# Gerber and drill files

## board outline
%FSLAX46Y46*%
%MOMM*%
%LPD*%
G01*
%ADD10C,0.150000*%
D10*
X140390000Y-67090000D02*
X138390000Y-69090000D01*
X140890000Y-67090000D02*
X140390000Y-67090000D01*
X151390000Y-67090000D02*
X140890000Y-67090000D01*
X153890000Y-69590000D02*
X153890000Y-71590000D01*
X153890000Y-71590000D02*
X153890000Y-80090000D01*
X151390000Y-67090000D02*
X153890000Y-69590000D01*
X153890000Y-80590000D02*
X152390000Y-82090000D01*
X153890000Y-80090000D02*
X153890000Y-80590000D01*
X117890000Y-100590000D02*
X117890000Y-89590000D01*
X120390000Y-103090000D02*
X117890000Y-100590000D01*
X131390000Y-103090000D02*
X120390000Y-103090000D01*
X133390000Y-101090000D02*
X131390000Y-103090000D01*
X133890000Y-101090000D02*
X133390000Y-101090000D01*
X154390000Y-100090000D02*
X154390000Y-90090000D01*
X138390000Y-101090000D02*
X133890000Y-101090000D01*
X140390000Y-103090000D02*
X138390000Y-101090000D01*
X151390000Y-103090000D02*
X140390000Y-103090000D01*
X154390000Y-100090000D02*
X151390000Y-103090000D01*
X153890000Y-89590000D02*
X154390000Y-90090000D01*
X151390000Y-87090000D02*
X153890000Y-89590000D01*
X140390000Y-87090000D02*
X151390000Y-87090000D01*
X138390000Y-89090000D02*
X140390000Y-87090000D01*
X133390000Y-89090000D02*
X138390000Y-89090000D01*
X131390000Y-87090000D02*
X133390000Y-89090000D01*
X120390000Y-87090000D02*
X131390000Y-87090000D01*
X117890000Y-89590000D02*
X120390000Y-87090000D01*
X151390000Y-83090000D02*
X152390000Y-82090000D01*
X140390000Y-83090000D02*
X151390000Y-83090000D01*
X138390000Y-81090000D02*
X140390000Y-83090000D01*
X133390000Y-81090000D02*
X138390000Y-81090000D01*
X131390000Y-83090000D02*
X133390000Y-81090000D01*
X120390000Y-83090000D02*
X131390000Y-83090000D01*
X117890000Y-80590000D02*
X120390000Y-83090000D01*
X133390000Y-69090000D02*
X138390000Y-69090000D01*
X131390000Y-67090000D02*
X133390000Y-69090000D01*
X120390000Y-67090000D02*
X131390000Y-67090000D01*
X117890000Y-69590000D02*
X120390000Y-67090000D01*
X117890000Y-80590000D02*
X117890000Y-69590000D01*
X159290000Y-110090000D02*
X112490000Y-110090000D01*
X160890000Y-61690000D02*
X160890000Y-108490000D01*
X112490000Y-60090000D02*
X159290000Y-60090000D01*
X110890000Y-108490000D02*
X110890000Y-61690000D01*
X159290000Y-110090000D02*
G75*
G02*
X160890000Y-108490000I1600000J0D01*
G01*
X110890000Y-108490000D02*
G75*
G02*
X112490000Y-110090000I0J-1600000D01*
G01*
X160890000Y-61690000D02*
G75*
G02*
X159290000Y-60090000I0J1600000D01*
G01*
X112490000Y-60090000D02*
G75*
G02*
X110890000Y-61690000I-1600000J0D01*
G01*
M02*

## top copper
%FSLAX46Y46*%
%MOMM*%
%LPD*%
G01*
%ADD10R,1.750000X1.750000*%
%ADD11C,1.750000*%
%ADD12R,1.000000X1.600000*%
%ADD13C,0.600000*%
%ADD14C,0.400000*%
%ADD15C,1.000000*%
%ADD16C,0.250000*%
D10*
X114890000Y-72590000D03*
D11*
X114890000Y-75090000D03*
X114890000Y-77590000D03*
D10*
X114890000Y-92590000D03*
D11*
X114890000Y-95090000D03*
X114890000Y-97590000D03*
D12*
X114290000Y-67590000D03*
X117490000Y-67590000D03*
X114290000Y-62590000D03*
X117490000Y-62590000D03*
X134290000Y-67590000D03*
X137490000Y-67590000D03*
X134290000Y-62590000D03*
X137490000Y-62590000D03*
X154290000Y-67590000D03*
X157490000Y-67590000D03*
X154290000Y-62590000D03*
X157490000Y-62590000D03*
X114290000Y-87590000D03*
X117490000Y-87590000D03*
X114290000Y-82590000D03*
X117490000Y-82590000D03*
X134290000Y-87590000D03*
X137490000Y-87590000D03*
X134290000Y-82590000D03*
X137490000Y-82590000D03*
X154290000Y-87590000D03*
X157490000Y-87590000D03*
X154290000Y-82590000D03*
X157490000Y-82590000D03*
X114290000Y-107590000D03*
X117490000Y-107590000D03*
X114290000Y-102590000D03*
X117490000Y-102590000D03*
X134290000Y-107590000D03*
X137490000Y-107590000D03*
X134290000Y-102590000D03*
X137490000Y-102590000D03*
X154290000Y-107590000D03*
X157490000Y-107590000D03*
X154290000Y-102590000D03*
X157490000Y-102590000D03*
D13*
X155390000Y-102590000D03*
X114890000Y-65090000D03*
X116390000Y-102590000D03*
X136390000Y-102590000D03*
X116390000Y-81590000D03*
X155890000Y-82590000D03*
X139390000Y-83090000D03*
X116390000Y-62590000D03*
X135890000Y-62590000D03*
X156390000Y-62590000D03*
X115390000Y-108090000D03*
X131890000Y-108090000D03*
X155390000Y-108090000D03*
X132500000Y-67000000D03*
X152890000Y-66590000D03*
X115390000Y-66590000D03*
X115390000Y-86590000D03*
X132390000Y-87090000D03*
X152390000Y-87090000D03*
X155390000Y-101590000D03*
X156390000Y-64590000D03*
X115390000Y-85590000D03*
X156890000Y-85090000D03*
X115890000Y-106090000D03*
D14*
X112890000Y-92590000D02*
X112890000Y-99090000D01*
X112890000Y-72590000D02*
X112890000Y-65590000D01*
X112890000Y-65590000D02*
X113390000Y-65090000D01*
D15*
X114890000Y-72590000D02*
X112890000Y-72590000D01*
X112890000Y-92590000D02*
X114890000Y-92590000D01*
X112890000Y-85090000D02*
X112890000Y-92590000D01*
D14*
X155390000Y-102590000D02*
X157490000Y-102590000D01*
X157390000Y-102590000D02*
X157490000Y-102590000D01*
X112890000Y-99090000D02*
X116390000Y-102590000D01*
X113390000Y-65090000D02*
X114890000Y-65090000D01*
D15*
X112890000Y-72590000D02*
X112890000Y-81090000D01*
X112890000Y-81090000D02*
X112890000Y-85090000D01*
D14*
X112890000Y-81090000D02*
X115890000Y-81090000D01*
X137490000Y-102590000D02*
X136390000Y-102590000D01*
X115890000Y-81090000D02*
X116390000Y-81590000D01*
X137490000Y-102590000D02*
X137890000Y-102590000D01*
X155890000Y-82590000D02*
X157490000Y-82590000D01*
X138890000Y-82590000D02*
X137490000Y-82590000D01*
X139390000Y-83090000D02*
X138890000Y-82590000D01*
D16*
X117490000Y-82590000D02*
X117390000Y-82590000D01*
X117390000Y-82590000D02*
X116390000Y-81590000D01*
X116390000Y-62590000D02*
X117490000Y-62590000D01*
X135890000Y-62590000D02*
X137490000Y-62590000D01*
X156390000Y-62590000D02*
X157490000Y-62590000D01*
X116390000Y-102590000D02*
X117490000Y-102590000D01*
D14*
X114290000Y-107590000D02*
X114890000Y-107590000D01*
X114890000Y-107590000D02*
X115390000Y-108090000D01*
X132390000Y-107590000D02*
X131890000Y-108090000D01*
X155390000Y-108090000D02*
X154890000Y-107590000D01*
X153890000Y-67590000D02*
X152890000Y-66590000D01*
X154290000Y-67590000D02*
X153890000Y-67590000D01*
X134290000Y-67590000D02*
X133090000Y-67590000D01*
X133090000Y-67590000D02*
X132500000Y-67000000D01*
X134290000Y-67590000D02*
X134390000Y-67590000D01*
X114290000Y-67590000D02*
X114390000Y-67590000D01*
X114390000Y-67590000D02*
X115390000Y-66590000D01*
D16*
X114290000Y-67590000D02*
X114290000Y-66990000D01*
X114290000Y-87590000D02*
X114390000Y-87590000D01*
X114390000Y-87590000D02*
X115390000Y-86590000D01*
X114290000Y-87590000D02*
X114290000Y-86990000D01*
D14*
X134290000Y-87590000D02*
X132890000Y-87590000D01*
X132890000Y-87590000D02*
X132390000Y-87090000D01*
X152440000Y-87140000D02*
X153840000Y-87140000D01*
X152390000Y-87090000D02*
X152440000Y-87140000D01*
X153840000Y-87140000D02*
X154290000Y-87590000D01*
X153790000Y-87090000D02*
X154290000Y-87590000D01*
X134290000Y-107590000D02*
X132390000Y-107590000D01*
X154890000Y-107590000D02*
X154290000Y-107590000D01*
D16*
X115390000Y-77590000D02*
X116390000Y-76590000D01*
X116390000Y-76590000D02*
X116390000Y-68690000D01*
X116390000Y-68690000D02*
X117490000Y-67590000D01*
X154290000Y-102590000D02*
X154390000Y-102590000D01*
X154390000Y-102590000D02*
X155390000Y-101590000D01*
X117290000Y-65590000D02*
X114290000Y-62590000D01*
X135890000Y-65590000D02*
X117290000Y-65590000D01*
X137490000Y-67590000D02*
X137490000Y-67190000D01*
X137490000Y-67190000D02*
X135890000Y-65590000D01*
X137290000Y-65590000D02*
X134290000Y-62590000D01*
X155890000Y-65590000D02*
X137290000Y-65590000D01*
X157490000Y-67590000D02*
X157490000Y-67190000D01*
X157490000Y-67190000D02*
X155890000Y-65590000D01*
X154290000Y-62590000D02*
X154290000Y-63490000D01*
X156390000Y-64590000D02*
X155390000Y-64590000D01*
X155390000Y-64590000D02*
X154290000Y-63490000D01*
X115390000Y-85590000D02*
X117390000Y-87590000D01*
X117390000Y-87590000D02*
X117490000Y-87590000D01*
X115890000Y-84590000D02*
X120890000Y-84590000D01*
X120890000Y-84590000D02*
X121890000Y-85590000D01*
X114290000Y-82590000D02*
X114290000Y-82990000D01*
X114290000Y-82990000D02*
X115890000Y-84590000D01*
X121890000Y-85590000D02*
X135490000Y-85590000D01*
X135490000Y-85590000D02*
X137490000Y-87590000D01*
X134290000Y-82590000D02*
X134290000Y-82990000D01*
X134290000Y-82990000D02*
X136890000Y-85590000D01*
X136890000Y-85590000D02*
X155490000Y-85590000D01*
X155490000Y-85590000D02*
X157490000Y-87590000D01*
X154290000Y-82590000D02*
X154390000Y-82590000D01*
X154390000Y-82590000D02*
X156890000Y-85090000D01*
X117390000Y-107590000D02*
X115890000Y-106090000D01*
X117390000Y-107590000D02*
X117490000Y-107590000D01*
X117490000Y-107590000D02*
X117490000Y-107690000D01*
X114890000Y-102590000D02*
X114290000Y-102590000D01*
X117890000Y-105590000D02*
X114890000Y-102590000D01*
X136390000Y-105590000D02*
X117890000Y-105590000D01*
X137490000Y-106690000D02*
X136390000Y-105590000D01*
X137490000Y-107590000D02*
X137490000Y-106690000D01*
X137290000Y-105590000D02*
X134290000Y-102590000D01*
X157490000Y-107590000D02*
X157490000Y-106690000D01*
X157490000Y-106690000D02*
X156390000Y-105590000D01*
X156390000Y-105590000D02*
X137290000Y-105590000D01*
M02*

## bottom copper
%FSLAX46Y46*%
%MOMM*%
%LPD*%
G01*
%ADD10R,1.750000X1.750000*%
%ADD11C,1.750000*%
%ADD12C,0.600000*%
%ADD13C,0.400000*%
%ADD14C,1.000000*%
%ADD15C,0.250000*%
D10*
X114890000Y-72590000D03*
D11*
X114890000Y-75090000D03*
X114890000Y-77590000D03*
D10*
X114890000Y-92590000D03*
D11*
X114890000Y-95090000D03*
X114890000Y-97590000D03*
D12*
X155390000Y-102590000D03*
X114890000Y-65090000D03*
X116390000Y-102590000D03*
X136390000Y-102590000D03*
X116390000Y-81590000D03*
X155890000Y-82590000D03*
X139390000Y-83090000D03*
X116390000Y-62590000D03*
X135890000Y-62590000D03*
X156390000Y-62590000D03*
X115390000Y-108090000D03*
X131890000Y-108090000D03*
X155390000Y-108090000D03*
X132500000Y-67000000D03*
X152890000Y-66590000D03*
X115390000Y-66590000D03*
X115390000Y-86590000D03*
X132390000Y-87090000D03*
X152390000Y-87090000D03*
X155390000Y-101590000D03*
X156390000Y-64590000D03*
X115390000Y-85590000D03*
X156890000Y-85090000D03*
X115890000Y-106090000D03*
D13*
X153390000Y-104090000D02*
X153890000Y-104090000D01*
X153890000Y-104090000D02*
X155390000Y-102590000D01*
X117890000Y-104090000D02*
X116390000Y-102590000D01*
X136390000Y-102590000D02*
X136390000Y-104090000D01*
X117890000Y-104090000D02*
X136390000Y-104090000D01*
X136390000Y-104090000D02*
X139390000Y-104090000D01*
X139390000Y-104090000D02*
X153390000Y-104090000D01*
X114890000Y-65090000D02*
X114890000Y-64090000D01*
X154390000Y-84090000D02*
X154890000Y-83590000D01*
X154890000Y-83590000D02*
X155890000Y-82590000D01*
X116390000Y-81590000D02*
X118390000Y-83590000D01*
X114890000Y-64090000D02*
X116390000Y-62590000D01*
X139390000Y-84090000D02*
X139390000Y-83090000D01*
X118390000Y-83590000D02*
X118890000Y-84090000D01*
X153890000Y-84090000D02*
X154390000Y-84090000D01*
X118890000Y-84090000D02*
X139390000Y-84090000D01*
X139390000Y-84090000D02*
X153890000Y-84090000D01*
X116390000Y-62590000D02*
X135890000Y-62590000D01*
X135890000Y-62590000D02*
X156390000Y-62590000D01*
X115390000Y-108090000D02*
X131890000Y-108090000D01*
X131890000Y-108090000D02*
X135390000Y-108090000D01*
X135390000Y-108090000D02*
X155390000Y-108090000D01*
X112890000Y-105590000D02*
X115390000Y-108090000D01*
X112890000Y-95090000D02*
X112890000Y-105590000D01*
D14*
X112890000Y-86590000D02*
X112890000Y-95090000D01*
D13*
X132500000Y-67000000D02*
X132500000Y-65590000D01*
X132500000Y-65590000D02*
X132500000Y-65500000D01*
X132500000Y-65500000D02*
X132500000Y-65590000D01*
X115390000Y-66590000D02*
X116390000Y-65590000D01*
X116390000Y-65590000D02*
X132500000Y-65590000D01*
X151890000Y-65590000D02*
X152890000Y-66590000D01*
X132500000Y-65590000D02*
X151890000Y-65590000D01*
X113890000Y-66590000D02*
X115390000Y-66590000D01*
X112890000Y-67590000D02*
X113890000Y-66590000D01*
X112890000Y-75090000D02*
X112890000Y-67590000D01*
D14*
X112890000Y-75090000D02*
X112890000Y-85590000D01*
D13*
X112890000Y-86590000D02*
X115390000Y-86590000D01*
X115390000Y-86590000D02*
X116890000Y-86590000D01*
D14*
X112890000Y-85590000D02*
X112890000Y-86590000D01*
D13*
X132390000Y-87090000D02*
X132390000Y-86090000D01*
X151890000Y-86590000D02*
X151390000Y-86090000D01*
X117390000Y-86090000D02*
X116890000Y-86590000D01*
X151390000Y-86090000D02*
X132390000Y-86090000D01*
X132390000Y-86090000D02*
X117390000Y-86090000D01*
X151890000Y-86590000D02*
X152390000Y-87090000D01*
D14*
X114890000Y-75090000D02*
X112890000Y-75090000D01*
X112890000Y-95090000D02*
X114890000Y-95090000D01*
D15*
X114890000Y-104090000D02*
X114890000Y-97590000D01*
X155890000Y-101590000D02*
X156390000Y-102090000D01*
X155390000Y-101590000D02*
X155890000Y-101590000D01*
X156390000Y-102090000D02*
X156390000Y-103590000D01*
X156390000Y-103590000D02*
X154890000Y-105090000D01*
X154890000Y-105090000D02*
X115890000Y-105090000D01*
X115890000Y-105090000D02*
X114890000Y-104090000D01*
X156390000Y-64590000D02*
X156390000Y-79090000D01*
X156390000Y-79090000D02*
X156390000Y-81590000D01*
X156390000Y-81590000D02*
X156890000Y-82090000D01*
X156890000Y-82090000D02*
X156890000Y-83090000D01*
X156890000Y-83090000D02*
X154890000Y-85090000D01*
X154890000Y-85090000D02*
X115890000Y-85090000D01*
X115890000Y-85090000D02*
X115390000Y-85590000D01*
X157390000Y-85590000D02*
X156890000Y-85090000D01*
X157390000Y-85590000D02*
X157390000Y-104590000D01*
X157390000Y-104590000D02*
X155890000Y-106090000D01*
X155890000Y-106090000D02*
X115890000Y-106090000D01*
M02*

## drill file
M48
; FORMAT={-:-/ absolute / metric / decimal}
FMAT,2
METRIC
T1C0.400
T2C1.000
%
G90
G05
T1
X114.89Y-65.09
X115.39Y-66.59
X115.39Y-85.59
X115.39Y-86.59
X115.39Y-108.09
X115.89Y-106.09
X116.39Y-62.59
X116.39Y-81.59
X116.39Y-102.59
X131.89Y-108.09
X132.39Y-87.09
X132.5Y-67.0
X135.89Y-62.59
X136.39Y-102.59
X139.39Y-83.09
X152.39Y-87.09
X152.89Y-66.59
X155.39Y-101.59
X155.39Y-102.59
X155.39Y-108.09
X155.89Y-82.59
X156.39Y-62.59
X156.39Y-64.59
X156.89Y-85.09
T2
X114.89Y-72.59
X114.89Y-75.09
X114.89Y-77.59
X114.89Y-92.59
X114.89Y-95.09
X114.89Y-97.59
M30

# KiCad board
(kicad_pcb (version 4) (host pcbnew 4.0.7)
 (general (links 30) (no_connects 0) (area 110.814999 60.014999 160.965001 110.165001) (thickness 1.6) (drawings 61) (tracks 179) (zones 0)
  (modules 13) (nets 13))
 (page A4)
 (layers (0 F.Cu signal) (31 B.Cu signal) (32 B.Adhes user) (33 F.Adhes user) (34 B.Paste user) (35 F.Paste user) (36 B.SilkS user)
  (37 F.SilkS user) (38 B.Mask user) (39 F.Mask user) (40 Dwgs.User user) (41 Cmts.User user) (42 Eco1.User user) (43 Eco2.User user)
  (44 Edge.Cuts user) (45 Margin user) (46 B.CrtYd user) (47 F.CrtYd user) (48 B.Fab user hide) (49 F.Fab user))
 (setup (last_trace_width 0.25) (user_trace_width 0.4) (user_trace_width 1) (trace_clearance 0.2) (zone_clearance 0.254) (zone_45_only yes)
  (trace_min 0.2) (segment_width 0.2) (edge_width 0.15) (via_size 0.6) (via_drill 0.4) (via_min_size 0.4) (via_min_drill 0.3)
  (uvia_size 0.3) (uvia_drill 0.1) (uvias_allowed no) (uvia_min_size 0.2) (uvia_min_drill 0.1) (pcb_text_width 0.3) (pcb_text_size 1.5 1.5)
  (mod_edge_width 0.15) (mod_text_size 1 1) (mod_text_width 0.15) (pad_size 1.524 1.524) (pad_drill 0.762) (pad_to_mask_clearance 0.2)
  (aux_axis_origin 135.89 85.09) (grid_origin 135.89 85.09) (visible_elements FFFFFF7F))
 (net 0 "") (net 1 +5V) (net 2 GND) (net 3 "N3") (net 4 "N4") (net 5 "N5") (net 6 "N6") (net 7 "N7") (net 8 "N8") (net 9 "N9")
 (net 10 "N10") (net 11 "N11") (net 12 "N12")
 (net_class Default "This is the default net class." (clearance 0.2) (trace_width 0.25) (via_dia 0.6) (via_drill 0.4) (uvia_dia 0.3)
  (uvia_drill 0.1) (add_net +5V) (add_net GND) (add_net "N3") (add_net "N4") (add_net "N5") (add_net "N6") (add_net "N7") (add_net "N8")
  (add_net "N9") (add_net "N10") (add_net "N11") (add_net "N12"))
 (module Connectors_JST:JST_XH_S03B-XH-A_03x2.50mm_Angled (layer F.Cu) (at 114.89 72.59 270)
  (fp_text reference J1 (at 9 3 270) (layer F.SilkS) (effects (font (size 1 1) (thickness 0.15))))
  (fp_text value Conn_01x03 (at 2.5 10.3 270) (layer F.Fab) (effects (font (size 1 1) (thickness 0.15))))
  (pad 1 thru_hole rect (at 0 0 270) (size 1.75 1.75) (drill 1) (layers *.Cu *.Mask F.SilkS) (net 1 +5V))
  (pad 2 thru_hole circle (at 2.5 0 270) (size 1.75 1.75) (drill 1) (layers *.Cu *.Mask F.SilkS) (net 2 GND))
  (pad 3 thru_hole circle (at 5 0 270) (size 1.75 1.75) (drill 1) (layers *.Cu *.Mask F.SilkS) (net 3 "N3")))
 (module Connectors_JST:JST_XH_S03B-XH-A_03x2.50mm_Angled (layer F.Cu) (at 114.89 92.59 270)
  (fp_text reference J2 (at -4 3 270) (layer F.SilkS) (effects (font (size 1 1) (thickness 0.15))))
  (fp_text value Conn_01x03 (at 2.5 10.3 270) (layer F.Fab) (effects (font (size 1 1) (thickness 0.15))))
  (pad 1 thru_hole rect (at 0 0 270) (size 1.75 1.75) (drill 1) (layers *.Cu *.Mask F.SilkS) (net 1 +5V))
  (pad 2 thru_hole circle (at 2.5 0 270) (size 1.75 1.75) (drill 1) (layers *.Cu *.Mask F.SilkS) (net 2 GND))
  (pad 3 thru_hole circle (at 5 0 270) (size 1.75 1.75) (drill 1) (layers *.Cu *.Mask F.SilkS) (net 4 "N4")))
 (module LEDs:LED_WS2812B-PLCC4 (layer F.Cu) (at 115.89 65.09 270)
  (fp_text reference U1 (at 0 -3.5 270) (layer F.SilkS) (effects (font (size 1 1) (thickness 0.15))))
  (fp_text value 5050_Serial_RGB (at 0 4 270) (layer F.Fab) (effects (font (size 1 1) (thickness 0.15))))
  (pad 3 smd rect (at 2.5 1.6 270) (size 1.6 1) (layers F.Cu F.Paste F.Mask) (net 2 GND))
  (pad 4 smd rect (at 2.5 -1.6 270) (size 1.6 1) (layers F.Cu F.Paste F.Mask) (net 3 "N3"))
  (pad 2 smd rect (at -2.5 1.6 270) (size 1.6 1) (layers F.Cu F.Paste F.Mask) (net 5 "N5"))
  (pad 1 smd rect (at -2.5 -1.6 270) (size 1.6 1) (layers F.Cu F.Paste F.Mask) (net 1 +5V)))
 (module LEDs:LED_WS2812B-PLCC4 (layer F.Cu) (at 135.89 65.09 270)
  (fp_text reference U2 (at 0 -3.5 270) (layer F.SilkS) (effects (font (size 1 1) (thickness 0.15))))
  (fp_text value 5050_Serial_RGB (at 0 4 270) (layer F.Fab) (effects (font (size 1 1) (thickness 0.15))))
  (pad 3 smd rect (at 2.5 1.6 270) (size 1.6 1) (layers F.Cu F.Paste F.Mask) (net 2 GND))
  (pad 4 smd rect (at 2.5 -1.6 270) (size 1.6 1) (layers F.Cu F.Paste F.Mask) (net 5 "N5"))
  (pad 2 smd rect (at -2.5 1.6 270) (size 1.6 1) (layers F.Cu F.Paste F.Mask) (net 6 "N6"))
  (pad 1 smd rect (at -2.5 -1.6 270) (size 1.6 1) (layers F.Cu F.Paste F.Mask) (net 1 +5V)))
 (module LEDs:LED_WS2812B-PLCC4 (layer F.Cu) (at 155.89 65.09 270)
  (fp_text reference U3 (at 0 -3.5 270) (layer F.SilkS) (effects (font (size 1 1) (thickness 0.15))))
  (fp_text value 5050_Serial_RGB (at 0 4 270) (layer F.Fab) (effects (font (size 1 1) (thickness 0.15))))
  (pad 3 smd rect (at 2.5 1.6 270) (size 1.6 1) (layers F.Cu F.Paste F.Mask) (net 2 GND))
  (pad 4 smd rect (at 2.5 -1.6 270) (size 1.6 1) (layers F.Cu F.Paste F.Mask) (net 6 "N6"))
  (pad 2 smd rect (at -2.5 1.6 270) (size 1.6 1) (layers F.Cu F.Paste F.Mask) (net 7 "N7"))
  (pad 1 smd rect (at -2.5 -1.6 270) (size 1.6 1) (layers F.Cu F.Paste F.Mask) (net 1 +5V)))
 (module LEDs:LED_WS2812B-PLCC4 (layer F.Cu) (at 115.89 85.09 270)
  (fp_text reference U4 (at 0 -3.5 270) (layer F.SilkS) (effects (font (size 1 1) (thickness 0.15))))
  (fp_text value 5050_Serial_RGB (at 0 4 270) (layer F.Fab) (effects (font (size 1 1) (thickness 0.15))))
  (pad 3 smd rect (at 2.5 1.6 270) (size 1.6 1) (layers F.Cu F.Paste F.Mask) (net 2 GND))
  (pad 4 smd rect (at 2.5 -1.6 270) (size 1.6 1) (layers F.Cu F.Paste F.Mask) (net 7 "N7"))
  (pad 2 smd rect (at -2.5 1.6 270) (size 1.6 1) (layers F.Cu F.Paste F.Mask) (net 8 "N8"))
  (pad 1 smd rect (at -2.5 -1.6 270) (size 1.6 1) (layers F.Cu F.Paste F.Mask) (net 1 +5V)))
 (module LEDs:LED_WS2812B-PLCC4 (layer F.Cu) (at 135.89 85.09 270)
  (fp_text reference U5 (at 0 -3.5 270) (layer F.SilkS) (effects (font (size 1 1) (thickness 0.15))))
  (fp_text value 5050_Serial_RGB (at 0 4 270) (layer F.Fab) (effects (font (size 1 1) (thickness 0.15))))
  (pad 3 smd rect (at 2.5 1.6 270) (size 1.6 1) (layers F.Cu F.Paste F.Mask) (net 2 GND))
  (pad 4 smd rect (at 2.5 -1.6 270) (size 1.6 1) (layers F.Cu F.Paste F.Mask) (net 8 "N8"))
  (pad 2 smd rect (at -2.5 1.6 270) (size 1.6 1) (layers F.Cu F.Paste F.Mask) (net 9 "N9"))
  (pad 1 smd rect (at -2.5 -1.6 270) (size 1.6 1) (layers F.Cu F.Paste F.Mask) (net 1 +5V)))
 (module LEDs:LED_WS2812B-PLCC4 (layer F.Cu) (at 155.89 85.09 270)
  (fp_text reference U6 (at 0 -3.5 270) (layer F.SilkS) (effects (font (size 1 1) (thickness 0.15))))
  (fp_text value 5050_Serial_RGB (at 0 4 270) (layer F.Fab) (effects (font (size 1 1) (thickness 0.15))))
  (pad 3 smd rect (at 2.5 1.6 270) (size 1.6 1) (layers F.Cu F.Paste F.Mask) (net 2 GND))
  (pad 4 smd rect (at 2.5 -1.6 270) (size 1.6 1) (layers F.Cu F.Paste F.Mask) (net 9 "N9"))
  (pad 2 smd rect (at -2.5 1.6 270) (size 1.6 1) (layers F.Cu F.Paste F.Mask) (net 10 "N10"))
  (pad 1 smd rect (at -2.5 -1.6 270) (size 1.6 1) (layers F.Cu F.Paste F.Mask) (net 1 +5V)))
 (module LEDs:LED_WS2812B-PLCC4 (layer F.Cu) (at 115.89 105.09 270)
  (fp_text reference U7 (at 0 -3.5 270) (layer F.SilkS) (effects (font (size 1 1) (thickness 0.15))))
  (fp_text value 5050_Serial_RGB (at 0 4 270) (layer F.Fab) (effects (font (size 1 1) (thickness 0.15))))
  (pad 3 smd rect (at 2.5 1.6 270) (size 1.6 1) (layers F.Cu F.Paste F.Mask) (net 2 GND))
  (pad 4 smd rect (at 2.5 -1.6 270) (size 1.6 1) (layers F.Cu F.Paste F.Mask) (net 10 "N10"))
  (pad 2 smd rect (at -2.5 1.6 270) (size 1.6 1) (layers F.Cu F.Paste F.Mask) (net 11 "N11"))
  (pad 1 smd rect (at -2.5 -1.6 270) (size 1.6 1) (layers F.Cu F.Paste F.Mask) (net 1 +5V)))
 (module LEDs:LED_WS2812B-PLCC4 (layer F.Cu) (at 135.89 105.09 270)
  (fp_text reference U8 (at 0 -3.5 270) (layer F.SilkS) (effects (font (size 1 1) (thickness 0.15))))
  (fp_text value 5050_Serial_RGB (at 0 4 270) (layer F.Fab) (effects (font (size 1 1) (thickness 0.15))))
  (pad 3 smd rect (at 2.5 1.6 270) (size 1.6 1) (layers F.Cu F.Paste F.Mask) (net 2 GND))
  (pad 4 smd rect (at 2.5 -1.6 270) (size 1.6 1) (layers F.Cu F.Paste F.Mask) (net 11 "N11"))
  (pad 2 smd rect (at -2.5 1.6 270) (size 1.6 1) (layers F.Cu F.Paste F.Mask) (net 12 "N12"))
  (pad 1 smd rect (at -2.5 -1.6 270) (size 1.6 1) (layers F.Cu F.Paste F.Mask) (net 1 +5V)))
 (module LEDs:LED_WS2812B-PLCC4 (layer F.Cu) (at 155.89 105.09 270)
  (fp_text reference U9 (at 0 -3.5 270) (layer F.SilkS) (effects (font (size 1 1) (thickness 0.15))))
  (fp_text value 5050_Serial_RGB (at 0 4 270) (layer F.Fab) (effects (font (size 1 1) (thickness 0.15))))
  (pad 3 smd rect (at 2.5 1.6 270) (size 1.6 1) (layers F.Cu F.Paste F.Mask) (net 2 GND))
  (pad 4 smd rect (at 2.5 -1.6 270) (size 1.6 1) (layers F.Cu F.Paste F.Mask) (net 12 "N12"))
  (pad 2 smd rect (at -2.5 1.6 270) (size 1.6 1) (layers F.Cu F.Paste F.Mask) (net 4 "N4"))
  (pad 1 smd rect (at -2.5 -1.6 270) (size 1.6 1) (layers F.Cu F.Paste F.Mask) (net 1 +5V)))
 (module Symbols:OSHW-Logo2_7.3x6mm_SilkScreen (layer F.Cu) (at 125.89 106.59)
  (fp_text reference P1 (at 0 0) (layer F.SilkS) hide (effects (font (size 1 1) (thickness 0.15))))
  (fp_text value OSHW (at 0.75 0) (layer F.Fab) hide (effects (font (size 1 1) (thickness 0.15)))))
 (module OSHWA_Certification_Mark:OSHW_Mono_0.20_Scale (layer F.Cu) (at 145.39 62.59)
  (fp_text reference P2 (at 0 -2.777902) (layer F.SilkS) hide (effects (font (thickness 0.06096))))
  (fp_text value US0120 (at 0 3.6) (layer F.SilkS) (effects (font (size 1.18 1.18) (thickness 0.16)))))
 (gr_line (start 140.39 67.09) (end 138.39 69.09) (angle 90) (layer Edge.Cuts) (width 0.15))
 (gr_line (start 140.89 67.09) (end 140.39 67.09) (angle 90) (layer Edge.Cuts) (width 0.15))
 (gr_line (start 151.39 67.09) (end 140.89 67.09) (angle 90) (layer Edge.Cuts) (width 0.15))
 (gr_line (start 153.89 69.59) (end 153.89 71.59) (angle 90) (layer Edge.Cuts) (width 0.15))
 (gr_line (start 153.89 71.59) (end 153.89 80.09) (angle 90) (layer Edge.Cuts) (width 0.15))
 (gr_line (start 151.39 67.09) (end 153.89 69.59) (angle 90) (layer Edge.Cuts) (width 0.15))
 (gr_line (start 153.89 80.59) (end 152.39 82.09) (angle 90) (layer Edge.Cuts) (width 0.15))
 (gr_line (start 153.89 80.09) (end 153.89 80.59) (angle 90) (layer Edge.Cuts) (width 0.15))
 (gr_line (start 117.89 100.59) (end 117.89 89.59) (angle 90) (layer Edge.Cuts) (width 0.15))
 (gr_line (start 120.39 103.09) (end 117.89 100.59) (angle 90) (layer Edge.Cuts) (width 0.15))
 (gr_line (start 131.39 103.09) (end 120.39 103.09) (angle 90) (layer Edge.Cuts) (width 0.15))
 (gr_line (start 133.39 101.09) (end 131.39 103.09) (angle 90) (layer Edge.Cuts) (width 0.15))
 (gr_line (start 133.89 101.09) (end 133.39 101.09) (angle 90) (layer Edge.Cuts) (width 0.15))
 (gr_line (start 154.39 100.09) (end 154.39 90.09) (angle 90) (layer Edge.Cuts) (width 0.15))
 (gr_line (start 138.39 101.09) (end 133.89 101.09) (angle 90) (layer Edge.Cuts) (width 0.15))
 (gr_line (start 140.39 103.09) (end 138.39 101.09) (angle 90) (layer Edge.Cuts) (width 0.15))
 (gr_line (start 151.39 103.09) (end 140.39 103.09) (angle 90) (layer Edge.Cuts) (width 0.15))
 (gr_line (start 154.39 100.09) (end 151.39 103.09) (angle 90) (layer Edge.Cuts) (width 0.15))
 (gr_line (start 153.89 89.59) (end 154.39 90.09) (angle 90) (layer Edge.Cuts) (width 0.15))
 (gr_line (start 151.39 87.09) (end 153.89 89.59) (angle 90) (layer Edge.Cuts) (width 0.15))
 (gr_line (start 140.39 87.09) (end 151.39 87.09) (angle 90) (layer Edge.Cuts) (width 0.15))
 (gr_line (start 138.39 89.09) (end 140.39 87.09) (angle 90) (layer Edge.Cuts) (width 0.15))
 (gr_line (start 133.39 89.09) (end 138.39 89.09) (angle 90) (layer Edge.Cuts) (width 0.15))
 (gr_line (start 131.39 87.09) (end 133.39 89.09) (angle 90) (layer Edge.Cuts) (width 0.15))
 (gr_line (start 120.39 87.09) (end 131.39 87.09) (angle 90) (layer Edge.Cuts) (width 0.15))
 (gr_line (start 117.89 89.59) (end 120.39 87.09) (angle 90) (layer Edge.Cuts) (width 0.15))
 (gr_line (start 151.39 83.09) (end 152.39 82.09) (angle 90) (layer Edge.Cuts) (width 0.15))
 (gr_line (start 140.39 83.09) (end 151.39 83.09) (angle 90) (layer Edge.Cuts) (width 0.15))
 (gr_line (start 138.39 81.09) (end 140.39 83.09) (angle 90) (layer Edge.Cuts) (width 0.15))
 (gr_line (start 133.39 81.09) (end 138.39 81.09) (angle 90) (layer Edge.Cuts) (width 0.15))
 (gr_line (start 131.39 83.09) (end 133.39 81.09) (angle 90) (layer Edge.Cuts) (width 0.15))
 (gr_line (start 120.39 83.09) (end 131.39 83.09) (angle 90) (layer Edge.Cuts) (width 0.15))
 (gr_line (start 117.89 80.59) (end 120.39 83.09) (angle 90) (layer Edge.Cuts) (width 0.15))
 (gr_line (start 133.39 69.09) (end 138.39 69.09) (angle 90) (layer Edge.Cuts) (width 0.15))
 (gr_line (start 131.39 67.09) (end 133.39 69.09) (angle 90) (layer Edge.Cuts) (width 0.15))
 (gr_line (start 120.39 67.09) (end 131.39 67.09) (angle 90) (layer Edge.Cuts) (width 0.15))
 (gr_line (start 117.89 69.59) (end 120.39 67.09) (angle 90) (layer Edge.Cuts) (width 0.15))
 (gr_line (start 117.89 80.59) (end 117.89 69.59) (angle 90) (layer Edge.Cuts) (width 0.15))
 (gr_line (start 159.29 110.09) (end 112.49 110.09) (angle 90) (layer Edge.Cuts) (width 0.15))
 (gr_line (start 160.89 61.69) (end 160.89 108.49) (angle 90) (layer Edge.Cuts) (width 0.15))
 (gr_line (start 112.49 60.09) (end 159.29 60.09) (angle 90) (layer Edge.Cuts) (width 0.15))
 (gr_line (start 110.89 108.49) (end 110.89 61.69) (angle 90) (layer Edge.Cuts) (width 0.15))
 (gr_arc (start 160.89 110.09) (end 159.29 110.09) (angle 90) (layer Edge.Cuts) (width 0.15))
 (gr_arc (start 110.89 110.09) (end 110.89 108.49) (angle 90) (layer Edge.Cuts) (width 0.15))
 (gr_arc (start 160.89 60.09) (end 160.89 61.69) (angle 90) (layer Edge.Cuts) (width 0.15))
 (gr_arc (start 110.89 60.09) (end 112.49 60.09) (angle 90) (layer Edge.Cuts) (width 0.15))
 (segment (start 112.89 92.59) (end 112.89 99.09) (width 0.4) (layer F.Cu) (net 1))
 (segment (start 112.89 72.59) (end 112.89 65.59) (width 0.4) (layer F.Cu) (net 1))
 (segment (start 112.89 65.59) (end 113.39 65.09) (width 0.4) (layer F.Cu) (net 1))
 (segment (start 114.89 72.59) (end 112.89 72.59) (width 1) (layer F.Cu) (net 1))
 (segment (start 112.89 92.59) (end 114.89 92.59) (width 1) (layer F.Cu) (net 1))
 (segment (start 112.89 85.09) (end 112.89 92.59) (width 1) (layer F.Cu) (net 1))
 (segment (start 153.39 104.09) (end 153.89 104.09) (width 0.4) (layer B.Cu) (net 1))
 (segment (start 155.39 102.59) (end 157.49 102.59) (width 0.4) (layer F.Cu) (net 1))
 (via (at 155.39 102.59) (size 0.6) (drill 0.4) (layers F.Cu B.Cu) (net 1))
 (segment (start 153.89 104.09) (end 155.39 102.59) (width 0.4) (layer B.Cu) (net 1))
 (segment (start 157.39 102.59) (end 157.49 102.59) (width 0.4) (layer F.Cu) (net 1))
 (segment (start 112.89 99.09) (end 116.39 102.59) (width 0.4) (layer F.Cu) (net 1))
 (segment (start 113.39 65.09) (end 114.89 65.09) (width 0.4) (layer F.Cu) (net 1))
 (segment (start 112.89 72.59) (end 112.89 81.09) (width 1) (layer F.Cu) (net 1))
 (segment (start 112.89 81.09) (end 112.89 85.09) (width 1) (layer F.Cu) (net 1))
 (segment (start 112.89 81.09) (end 115.89 81.09) (width 0.4) (layer F.Cu) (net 1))
 (via (at 114.89 65.09) (size 0.6) (drill 0.4) (layers F.Cu B.Cu) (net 1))
 (via (at 116.39 102.59) (size 0.6) (drill 0.4) (layers F.Cu B.Cu) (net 1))
 (segment (start 117.89 104.09) (end 116.39 102.59) (width 0.4) (layer B.Cu) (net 1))
 (segment (start 137.49 102.59) (end 136.39 102.59) (width 0.4) (layer F.Cu) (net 1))
 (segment (start 136.39 102.59) (end 136.39 104.09) (width 0.4) (layer B.Cu) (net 1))
 (via (at 136.39 102.59) (size 0.6) (drill 0.4) (layers F.Cu B.Cu) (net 1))
 (segment (start 115.89 81.09) (end 116.39 81.59) (width 0.4) (layer F.Cu) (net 1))
 (segment (start 137.49 102.59) (end 137.89 102.59) (width 0.4) (layer F.Cu) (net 1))
 (segment (start 117.89 104.09) (end 136.39 104.09) (width 0.4) (layer B.Cu) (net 1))
 (segment (start 136.39 104.09) (end 139.39 104.09) (width 0.4) (layer B.Cu) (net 1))
 (segment (start 139.39 104.09) (end 153.39 104.09) (width 0.4) (layer B.Cu) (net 1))
 (segment (start 114.89 65.09) (end 114.89 64.09) (width 0.4) (layer B.Cu) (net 1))
 (segment (start 154.39 84.09) (end 154.89 83.59) (width 0.4) (layer B.Cu) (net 1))
 (via (at 116.39 81.59) (size 0.6) (drill 0.4) (layers F.Cu B.Cu) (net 1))
 (segment (start 155.89 82.59) (end 157.49 82.59) (width 0.4) (layer F.Cu) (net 1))
 (segment (start 154.89 83.59) (end 155.89 82.59) (width 0.4) (layer B.Cu) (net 1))
 (via (at 155.89 82.59) (size 0.6) (drill 0.4) (layers F.Cu B.Cu) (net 1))
 (segment (start 116.39 81.59) (end 118.39 83.59) (width 0.4) (layer B.Cu) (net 1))
 (segment (start 114.89 64.09) (end 116.39 62.59) (width 0.4) (layer B.Cu) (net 1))
 (segment (start 139.39 84.09) (end 139.39 83.09) (width 0.4) (layer B.Cu) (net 1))
 (segment (start 138.89 82.59) (end 137.49 82.59) (width 0.4) (layer F.Cu) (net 1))
 (segment (start 139.39 83.09) (end 138.89 82.59) (width 0.4) (layer F.Cu) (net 1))
 (via (at 139.39 83.09) (size 0.6) (drill 0.4) (layers F.Cu B.Cu) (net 1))
 (segment (start 118.39 83.59) (end 118.89 84.09) (width 0.4) (layer B.Cu) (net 1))
 (segment (start 153.89 84.09) (end 154.39 84.09) (width 0.4) (layer B.Cu) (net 1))
 (segment (start 118.89 84.09) (end 139.39 84.09) (width 0.4) (layer B.Cu) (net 1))
 (segment (start 139.39 84.09) (end 153.89 84.09) (width 0.4) (layer B.Cu) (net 1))
 (segment (start 116.39 62.59) (end 135.89 62.59) (width 0.4) (layer B.Cu) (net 1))
 (via (at 116.39 62.59) (size 0.6) (drill 0.4) (layers F.Cu B.Cu) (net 1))
 (via (at 135.89 62.59) (size 0.6) (drill 0.4) (layers F.Cu B.Cu) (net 1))
 (segment (start 135.89 62.59) (end 156.39 62.59) (width 0.4) (layer B.Cu) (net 1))
 (via (at 156.39 62.59) (size 0.6) (drill 0.4) (layers F.Cu B.Cu) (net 1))
 (segment (start 117.49 82.59) (end 117.39 82.59) (width 0.25) (layer F.Cu) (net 1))
 (segment (start 117.39 82.59) (end 116.39 81.59) (width 0.25) (layer F.Cu) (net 1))
 (segment (start 116.39 62.59) (end 117.49 62.59) (width 0.25) (layer F.Cu) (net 1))
 (segment (start 135.89 62.59) (end 137.49 62.59) (width 0.25) (layer F.Cu) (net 1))
 (segment (start 156.39 62.59) (end 157.49 62.59) (width 0.25) (layer F.Cu) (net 1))
 (segment (start 116.39 102.59) (end 117.49 102.59) (width 0.25) (layer F.Cu) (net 1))
 (segment (start 114.29 107.59) (end 114.89 107.59) (width 0.4) (layer F.Cu) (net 2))
 (segment (start 114.89 107.59) (end 115.39 108.09) (width 0.4) (layer F.Cu) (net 2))
 (via (at 115.39 108.09) (size 0.6) (drill 0.4) (layers F.Cu B.Cu) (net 2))
 (via (at 131.89 108.09) (size 0.6) (drill 0.4) (layers F.Cu B.Cu) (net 2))
 (segment (start 115.39 108.09) (end 131.89 108.09) (width 0.4) (layer B.Cu) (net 2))
 (segment (start 131.89 108.09) (end 135.39 108.09) (width 0.4) (layer B.Cu) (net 2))
 (segment (start 135.39 108.09) (end 155.39 108.09) (width 0.4) (layer B.Cu) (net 2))
 (via (at 155.39 108.09) (size 0.6) (drill 0.4) (layers F.Cu B.Cu) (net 2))
 (segment (start 112.89 105.59) (end 115.39 108.09) (width 0.4) (layer B.Cu) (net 2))
 (segment (start 132.39 107.59) (end 131.89 108.09) (width 0.4) (layer F.Cu) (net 2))
 (segment (start 155.39 108.09) (end 154.89 107.59) (width 0.4) (layer F.Cu) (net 2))
 (segment (start 112.89 95.09) (end 112.89 105.59) (width 0.4) (layer B.Cu) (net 2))
 (segment (start 112.89 86.59) (end 112.89 95.09) (width 1) (layer B.Cu) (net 2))
 (segment (start 153.89 67.59) (end 152.89 66.59) (width 0.4) (layer F.Cu) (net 2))
 (segment (start 154.29 67.59) (end 153.89 67.59) (width 0.4) (layer F.Cu) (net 2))
 (segment (start 134.29 67.59) (end 133.09 67.59) (width 0.4) (layer F.Cu) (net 2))
 (segment (start 132.5 67) (end 132.5 65.59) (width 0.4) (layer B.Cu) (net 2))
 (via (at 132.5 67) (size 0.6) (drill 0.4) (layers F.Cu B.Cu) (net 2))
 (segment (start 133.09 67.59) (end 132.5 67) (width 0.4) (layer F.Cu) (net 2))
 (segment (start 132.5 65.59) (end 132.5 65.5) (width 0.4) (layer B.Cu) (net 2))
 (segment (start 132.5 65.5) (end 132.5 65.59) (width 0.4) (layer B.Cu) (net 2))
 (segment (start 115.39 66.59) (end 116.39 65.59) (width 0.4) (layer B.Cu) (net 2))
 (segment (start 116.39 65.59) (end 132.5 65.59) (width 0.4) (layer B.Cu) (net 2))
 (segment (start 151.89 65.59) (end 152.89 66.59) (width 0.4) (layer B.Cu) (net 2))
 (via (at 152.89 66.59) (size 0.6) (drill 0.4) (layers F.Cu B.Cu) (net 2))
 (segment (start 132.5 65.59) (end 151.89 65.59) (width 0.4) (layer B.Cu) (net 2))
 (segment (start 134.29 67.59) (end 134.39 67.59) (width 0.4) (layer F.Cu) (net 2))
 (via (at 115.39 66.59) (size 0.6) (drill 0.4) (layers F.Cu B.Cu) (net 2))
 (segment (start 113.89 66.59) (end 115.39 66.59) (width 0.4) (layer B.Cu) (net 2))
 (segment (start 112.89 67.59) (end 113.89 66.59) (width 0.4) (layer B.Cu) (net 2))
 (segment (start 112.89 75.09) (end 112.89 67.59) (width 0.4) (layer B.Cu) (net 2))
 (segment (start 112.89 75.09) (end 112.89 85.59) (width 1) (layer B.Cu) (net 2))
 (segment (start 114.29 67.59) (end 114.39 67.59) (width 0.4) (layer F.Cu) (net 2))
 (segment (start 114.39 67.59) (end 115.39 66.59) (width 0.4) (layer F.Cu) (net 2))
 (segment (start 114.29 67.59) (end 114.29 66.99) (width 0.25) (layer F.Cu) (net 2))
 (segment (start 114.29 87.59) (end 114.39 87.59) (width 0.25) (layer F.Cu) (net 2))
 (segment (start 114.39 87.59) (end 115.39 86.59) (width 0.25) (layer F.Cu) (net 2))
 (via (at 115.39 86.59) (size 0.6) (drill 0.4) (layers F.Cu B.Cu) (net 2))
 (segment (start 112.89 86.59) (end 115.39 86.59) (width 0.4) (layer B.Cu) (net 2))
 (segment (start 115.39 86.59) (end 116.89 86.59) (width 0.4) (layer B.Cu) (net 2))
 (segment (start 112.89 85.59) (end 112.89 86.59) (width 1) (layer B.Cu) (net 2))
 (segment (start 114.29 87.59) (end 114.29 86.99) (width 0.25) (layer F.Cu) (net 2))
 (segment (start 134.29 87.59) (end 132.89 87.59) (width 0.4) (layer F.Cu) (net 2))
 (segment (start 132.39 87.09) (end 132.39 86.09) (width 0.4) (layer B.Cu) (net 2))
 (via (at 132.39 87.09) (size 0.6) (drill 0.4) (layers F.Cu B.Cu) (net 2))
 (segment (start 132.89 87.59) (end 132.39 87.09) (width 0.4) (layer F.Cu) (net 2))
 (segment (start 151.89 86.59) (end 151.39 86.09) (width 0.4) (layer B.Cu) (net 2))
 (segment (start 117.39 86.09) (end 116.89 86.59) (width 0.4) (layer B.Cu) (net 2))
 (segment (start 151.39 86.09) (end 132.39 86.09) (width 0.4) (layer B.Cu) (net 2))
 (segment (start 132.39 86.09) (end 117.39 86.09) (width 0.4) (layer B.Cu) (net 2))
 (segment (start 152.44 87.14) (end 153.84 87.14) (width 0.4) (layer F.Cu) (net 2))
 (segment (start 152.39 87.09) (end 152.44 87.14) (width 0.4) (layer F.Cu) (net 2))
 (via (at 152.39 87.09) (size 0.6) (drill 0.4) (layers F.Cu B.Cu) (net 2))
 (segment (start 151.89 86.59) (end 152.39 87.09) (width 0.4) (layer B.Cu) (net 2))
 (segment (start 153.84 87.14) (end 154.29 87.59) (width 0.4) (layer F.Cu) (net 2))
 (segment (start 153.79 87.09) (end 154.29 87.59) (width 0.4) (layer F.Cu) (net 2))
 (segment (start 134.29 107.59) (end 132.39 107.59) (width 0.4) (layer F.Cu) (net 2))
 (segment (start 154.89 107.59) (end 154.29 107.59) (width 0.4) (layer F.Cu) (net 2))
 (segment (start 114.89 75.09) (end 112.89 75.09) (width 1) (layer B.Cu) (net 2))
 (segment (start 112.89 95.09) (end 114.89 95.09) (width 1) (layer B.Cu) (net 2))
 (segment (start 115.39 77.59) (end 116.39 76.59) (width 0.25) (layer F.Cu) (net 3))
 (segment (start 116.39 76.59) (end 116.39 68.69) (width 0.25) (layer F.Cu) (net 3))
 (segment (start 116.39 68.69) (end 117.49 67.59) (width 0.25) (layer F.Cu) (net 3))
 (segment (start 114.89 104.09) (end 114.89 97.59) (width 0.25) (layer B.Cu) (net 4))
 (segment (start 155.89 101.59) (end 156.39 102.09) (width 0.25) (layer B.Cu) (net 4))
 (segment (start 154.29 102.59) (end 154.39 102.59) (width 0.25) (layer F.Cu) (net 4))
 (segment (start 154.39 102.59) (end 155.39 101.59) (width 0.25) (layer F.Cu) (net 4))
 (via (at 155.39 101.59) (size 0.6) (drill 0.4) (layers F.Cu B.Cu) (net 4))
 (segment (start 155.39 101.59) (end 155.89 101.59) (width 0.25) (layer B.Cu) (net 4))
 (segment (start 156.39 102.09) (end 156.39 103.59) (width 0.25) (layer B.Cu) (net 4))
 (segment (start 156.39 103.59) (end 154.89 105.09) (width 0.25) (layer B.Cu) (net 4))
 (segment (start 154.89 105.09) (end 115.89 105.09) (width 0.25) (layer B.Cu) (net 4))
 (segment (start 115.89 105.09) (end 114.89 104.09) (width 0.25) (layer B.Cu) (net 4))
 (segment (start 117.29 65.59) (end 114.29 62.59) (width 0.25) (layer F.Cu) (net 5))
 (segment (start 135.89 65.59) (end 117.29 65.59) (width 0.25) (layer F.Cu) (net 5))
 (segment (start 137.49 67.59) (end 137.49 67.19) (width 0.25) (layer F.Cu) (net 5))
 (segment (start 137.49 67.19) (end 135.89 65.59) (width 0.25) (layer F.Cu) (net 5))
 (segment (start 137.29 65.59) (end 134.29 62.59) (width 0.25) (layer F.Cu) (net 6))
 (segment (start 155.89 65.59) (end 137.29 65.59) (width 0.25) (layer F.Cu) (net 6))
 (segment (start 157.49 67.59) (end 157.49 67.19) (width 0.25) (layer F.Cu) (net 6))
 (segment (start 157.49 67.19) (end 155.89 65.59) (width 0.25) (layer F.Cu) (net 6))
 (via (at 156.39 64.59) (size 0.6) (drill 0.4) (layers F.Cu B.Cu) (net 7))
 (segment (start 156.39 64.59) (end 156.39 79.09) (width 0.25) (layer B.Cu) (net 7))
 (segment (start 154.29 62.59) (end 154.29 63.49) (width 0.25) (layer F.Cu) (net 7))
 (segment (start 156.39 64.59) (end 155.39 64.59) (width 0.25) (layer F.Cu) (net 7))
 (segment (start 155.39 64.59) (end 154.29 63.49) (width 0.25) (layer F.Cu) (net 7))
 (segment (start 156.39 79.09) (end 156.39 81.59) (width 0.25) (layer B.Cu) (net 7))
 (segment (start 156.39 81.59) (end 156.89 82.09) (width 0.25) (layer B.Cu) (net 7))
 (segment (start 156.89 82.09) (end 156.89 83.09) (width 0.25) (layer B.Cu) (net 7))
 (via (at 115.39 85.59) (size 0.6) (drill 0.4) (layers F.Cu B.Cu) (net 7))
 (segment (start 156.89 83.09) (end 154.89 85.09) (width 0.25) (layer B.Cu) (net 7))
 (segment (start 154.89 85.09) (end 115.89 85.09) (width 0.25) (layer B.Cu) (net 7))
 (segment (start 115.89 85.09) (end 115.39 85.59) (width 0.25) (layer B.Cu) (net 7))
 (segment (start 115.39 85.59) (end 117.39 87.59) (width 0.25) (layer F.Cu) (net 7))
 (segment (start 117.39 87.59) (end 117.49 87.59) (width 0.25) (layer F.Cu) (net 7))
 (segment (start 115.89 84.59) (end 120.89 84.59) (width 0.25) (layer F.Cu) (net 8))
 (segment (start 120.89 84.59) (end 121.89 85.59) (width 0.25) (layer F.Cu) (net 8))
 (segment (start 114.29 82.59) (end 114.29 82.99) (width 0.25) (layer F.Cu) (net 8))
 (segment (start 114.29 82.99) (end 115.89 84.59) (width 0.25) (layer F.Cu) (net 8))
 (segment (start 121.89 85.59) (end 135.49 85.59) (width 0.25) (layer F.Cu) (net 8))
 (segment (start 135.49 85.59) (end 137.49 87.59) (width 0.25) (layer F.Cu) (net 8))
 (segment (start 134.29 82.59) (end 134.29 82.99) (width 0.25) (layer F.Cu) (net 9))
 (segment (start 134.29 82.99) (end 136.89 85.59) (width 0.25) (layer F.Cu) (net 9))
 (segment (start 136.89 85.59) (end 155.49 85.59) (width 0.25) (layer F.Cu) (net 9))
 (segment (start 155.49 85.59) (end 157.49 87.59) (width 0.25) (layer F.Cu) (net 9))
 (via (at 156.89 85.09) (size 0.6) (drill 0.4) (layers F.Cu B.Cu) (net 10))
 (segment (start 157.39 85.59) (end 156.89 85.09) (width 0.25) (layer B.Cu) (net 10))
 (segment (start 154.29 82.59) (end 154.39 82.59) (width 0.25) (layer F.Cu) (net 10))
 (segment (start 154.39 82.59) (end 156.89 85.09) (width 0.25) (layer F.Cu) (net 10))
 (segment (start 157.39 85.59) (end 157.39 104.59) (width 0.25) (layer B.Cu) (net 10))
 (segment (start 157.39 104.59) (end 155.89 106.09) (width 0.25) (layer B.Cu) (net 10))
 (segment (start 155.89 106.09) (end 115.89 106.09) (width 0.25) (layer B.Cu) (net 10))
 (via (at 115.89 106.09) (size 0.6) (drill 0.4) (layers F.Cu B.Cu) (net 10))
 (segment (start 117.39 107.59) (end 115.89 106.09) (width 0.25) (layer F.Cu) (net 10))
 (segment (start 117.39 107.59) (end 117.49 107.59) (width 0.25) (layer F.Cu) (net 10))
 (segment (start 117.49 107.59) (end 117.49 107.69) (width 0.25) (layer F.Cu) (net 10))
 (segment (start 114.89 102.59) (end 114.29 102.59) (width 0.25) (layer F.Cu) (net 11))
 (segment (start 117.89 105.59) (end 114.89 102.59) (width 0.25) (layer F.Cu) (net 11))
 (segment (start 136.39 105.59) (end 117.89 105.59) (width 0.25) (layer F.Cu) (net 11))
 (segment (start 137.49 106.69) (end 136.39 105.59) (width 0.25) (layer F.Cu) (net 11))
 (segment (start 137.49 107.59) (end 137.49 106.69) (width 0.25) (layer F.Cu) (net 11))
 (segment (start 137.29 105.59) (end 134.29 102.59) (width 0.25) (layer F.Cu) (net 12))
 (segment (start 157.49 107.59) (end 157.49 106.69) (width 0.25) (layer F.Cu) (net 12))
 (segment (start 157.49 106.69) (end 156.39 105.59) (width 0.25) (layer F.Cu) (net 12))
 (segment (start 156.39 105.59) (end 137.29 105.59) (width 0.25) (layer F.Cu) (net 12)))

